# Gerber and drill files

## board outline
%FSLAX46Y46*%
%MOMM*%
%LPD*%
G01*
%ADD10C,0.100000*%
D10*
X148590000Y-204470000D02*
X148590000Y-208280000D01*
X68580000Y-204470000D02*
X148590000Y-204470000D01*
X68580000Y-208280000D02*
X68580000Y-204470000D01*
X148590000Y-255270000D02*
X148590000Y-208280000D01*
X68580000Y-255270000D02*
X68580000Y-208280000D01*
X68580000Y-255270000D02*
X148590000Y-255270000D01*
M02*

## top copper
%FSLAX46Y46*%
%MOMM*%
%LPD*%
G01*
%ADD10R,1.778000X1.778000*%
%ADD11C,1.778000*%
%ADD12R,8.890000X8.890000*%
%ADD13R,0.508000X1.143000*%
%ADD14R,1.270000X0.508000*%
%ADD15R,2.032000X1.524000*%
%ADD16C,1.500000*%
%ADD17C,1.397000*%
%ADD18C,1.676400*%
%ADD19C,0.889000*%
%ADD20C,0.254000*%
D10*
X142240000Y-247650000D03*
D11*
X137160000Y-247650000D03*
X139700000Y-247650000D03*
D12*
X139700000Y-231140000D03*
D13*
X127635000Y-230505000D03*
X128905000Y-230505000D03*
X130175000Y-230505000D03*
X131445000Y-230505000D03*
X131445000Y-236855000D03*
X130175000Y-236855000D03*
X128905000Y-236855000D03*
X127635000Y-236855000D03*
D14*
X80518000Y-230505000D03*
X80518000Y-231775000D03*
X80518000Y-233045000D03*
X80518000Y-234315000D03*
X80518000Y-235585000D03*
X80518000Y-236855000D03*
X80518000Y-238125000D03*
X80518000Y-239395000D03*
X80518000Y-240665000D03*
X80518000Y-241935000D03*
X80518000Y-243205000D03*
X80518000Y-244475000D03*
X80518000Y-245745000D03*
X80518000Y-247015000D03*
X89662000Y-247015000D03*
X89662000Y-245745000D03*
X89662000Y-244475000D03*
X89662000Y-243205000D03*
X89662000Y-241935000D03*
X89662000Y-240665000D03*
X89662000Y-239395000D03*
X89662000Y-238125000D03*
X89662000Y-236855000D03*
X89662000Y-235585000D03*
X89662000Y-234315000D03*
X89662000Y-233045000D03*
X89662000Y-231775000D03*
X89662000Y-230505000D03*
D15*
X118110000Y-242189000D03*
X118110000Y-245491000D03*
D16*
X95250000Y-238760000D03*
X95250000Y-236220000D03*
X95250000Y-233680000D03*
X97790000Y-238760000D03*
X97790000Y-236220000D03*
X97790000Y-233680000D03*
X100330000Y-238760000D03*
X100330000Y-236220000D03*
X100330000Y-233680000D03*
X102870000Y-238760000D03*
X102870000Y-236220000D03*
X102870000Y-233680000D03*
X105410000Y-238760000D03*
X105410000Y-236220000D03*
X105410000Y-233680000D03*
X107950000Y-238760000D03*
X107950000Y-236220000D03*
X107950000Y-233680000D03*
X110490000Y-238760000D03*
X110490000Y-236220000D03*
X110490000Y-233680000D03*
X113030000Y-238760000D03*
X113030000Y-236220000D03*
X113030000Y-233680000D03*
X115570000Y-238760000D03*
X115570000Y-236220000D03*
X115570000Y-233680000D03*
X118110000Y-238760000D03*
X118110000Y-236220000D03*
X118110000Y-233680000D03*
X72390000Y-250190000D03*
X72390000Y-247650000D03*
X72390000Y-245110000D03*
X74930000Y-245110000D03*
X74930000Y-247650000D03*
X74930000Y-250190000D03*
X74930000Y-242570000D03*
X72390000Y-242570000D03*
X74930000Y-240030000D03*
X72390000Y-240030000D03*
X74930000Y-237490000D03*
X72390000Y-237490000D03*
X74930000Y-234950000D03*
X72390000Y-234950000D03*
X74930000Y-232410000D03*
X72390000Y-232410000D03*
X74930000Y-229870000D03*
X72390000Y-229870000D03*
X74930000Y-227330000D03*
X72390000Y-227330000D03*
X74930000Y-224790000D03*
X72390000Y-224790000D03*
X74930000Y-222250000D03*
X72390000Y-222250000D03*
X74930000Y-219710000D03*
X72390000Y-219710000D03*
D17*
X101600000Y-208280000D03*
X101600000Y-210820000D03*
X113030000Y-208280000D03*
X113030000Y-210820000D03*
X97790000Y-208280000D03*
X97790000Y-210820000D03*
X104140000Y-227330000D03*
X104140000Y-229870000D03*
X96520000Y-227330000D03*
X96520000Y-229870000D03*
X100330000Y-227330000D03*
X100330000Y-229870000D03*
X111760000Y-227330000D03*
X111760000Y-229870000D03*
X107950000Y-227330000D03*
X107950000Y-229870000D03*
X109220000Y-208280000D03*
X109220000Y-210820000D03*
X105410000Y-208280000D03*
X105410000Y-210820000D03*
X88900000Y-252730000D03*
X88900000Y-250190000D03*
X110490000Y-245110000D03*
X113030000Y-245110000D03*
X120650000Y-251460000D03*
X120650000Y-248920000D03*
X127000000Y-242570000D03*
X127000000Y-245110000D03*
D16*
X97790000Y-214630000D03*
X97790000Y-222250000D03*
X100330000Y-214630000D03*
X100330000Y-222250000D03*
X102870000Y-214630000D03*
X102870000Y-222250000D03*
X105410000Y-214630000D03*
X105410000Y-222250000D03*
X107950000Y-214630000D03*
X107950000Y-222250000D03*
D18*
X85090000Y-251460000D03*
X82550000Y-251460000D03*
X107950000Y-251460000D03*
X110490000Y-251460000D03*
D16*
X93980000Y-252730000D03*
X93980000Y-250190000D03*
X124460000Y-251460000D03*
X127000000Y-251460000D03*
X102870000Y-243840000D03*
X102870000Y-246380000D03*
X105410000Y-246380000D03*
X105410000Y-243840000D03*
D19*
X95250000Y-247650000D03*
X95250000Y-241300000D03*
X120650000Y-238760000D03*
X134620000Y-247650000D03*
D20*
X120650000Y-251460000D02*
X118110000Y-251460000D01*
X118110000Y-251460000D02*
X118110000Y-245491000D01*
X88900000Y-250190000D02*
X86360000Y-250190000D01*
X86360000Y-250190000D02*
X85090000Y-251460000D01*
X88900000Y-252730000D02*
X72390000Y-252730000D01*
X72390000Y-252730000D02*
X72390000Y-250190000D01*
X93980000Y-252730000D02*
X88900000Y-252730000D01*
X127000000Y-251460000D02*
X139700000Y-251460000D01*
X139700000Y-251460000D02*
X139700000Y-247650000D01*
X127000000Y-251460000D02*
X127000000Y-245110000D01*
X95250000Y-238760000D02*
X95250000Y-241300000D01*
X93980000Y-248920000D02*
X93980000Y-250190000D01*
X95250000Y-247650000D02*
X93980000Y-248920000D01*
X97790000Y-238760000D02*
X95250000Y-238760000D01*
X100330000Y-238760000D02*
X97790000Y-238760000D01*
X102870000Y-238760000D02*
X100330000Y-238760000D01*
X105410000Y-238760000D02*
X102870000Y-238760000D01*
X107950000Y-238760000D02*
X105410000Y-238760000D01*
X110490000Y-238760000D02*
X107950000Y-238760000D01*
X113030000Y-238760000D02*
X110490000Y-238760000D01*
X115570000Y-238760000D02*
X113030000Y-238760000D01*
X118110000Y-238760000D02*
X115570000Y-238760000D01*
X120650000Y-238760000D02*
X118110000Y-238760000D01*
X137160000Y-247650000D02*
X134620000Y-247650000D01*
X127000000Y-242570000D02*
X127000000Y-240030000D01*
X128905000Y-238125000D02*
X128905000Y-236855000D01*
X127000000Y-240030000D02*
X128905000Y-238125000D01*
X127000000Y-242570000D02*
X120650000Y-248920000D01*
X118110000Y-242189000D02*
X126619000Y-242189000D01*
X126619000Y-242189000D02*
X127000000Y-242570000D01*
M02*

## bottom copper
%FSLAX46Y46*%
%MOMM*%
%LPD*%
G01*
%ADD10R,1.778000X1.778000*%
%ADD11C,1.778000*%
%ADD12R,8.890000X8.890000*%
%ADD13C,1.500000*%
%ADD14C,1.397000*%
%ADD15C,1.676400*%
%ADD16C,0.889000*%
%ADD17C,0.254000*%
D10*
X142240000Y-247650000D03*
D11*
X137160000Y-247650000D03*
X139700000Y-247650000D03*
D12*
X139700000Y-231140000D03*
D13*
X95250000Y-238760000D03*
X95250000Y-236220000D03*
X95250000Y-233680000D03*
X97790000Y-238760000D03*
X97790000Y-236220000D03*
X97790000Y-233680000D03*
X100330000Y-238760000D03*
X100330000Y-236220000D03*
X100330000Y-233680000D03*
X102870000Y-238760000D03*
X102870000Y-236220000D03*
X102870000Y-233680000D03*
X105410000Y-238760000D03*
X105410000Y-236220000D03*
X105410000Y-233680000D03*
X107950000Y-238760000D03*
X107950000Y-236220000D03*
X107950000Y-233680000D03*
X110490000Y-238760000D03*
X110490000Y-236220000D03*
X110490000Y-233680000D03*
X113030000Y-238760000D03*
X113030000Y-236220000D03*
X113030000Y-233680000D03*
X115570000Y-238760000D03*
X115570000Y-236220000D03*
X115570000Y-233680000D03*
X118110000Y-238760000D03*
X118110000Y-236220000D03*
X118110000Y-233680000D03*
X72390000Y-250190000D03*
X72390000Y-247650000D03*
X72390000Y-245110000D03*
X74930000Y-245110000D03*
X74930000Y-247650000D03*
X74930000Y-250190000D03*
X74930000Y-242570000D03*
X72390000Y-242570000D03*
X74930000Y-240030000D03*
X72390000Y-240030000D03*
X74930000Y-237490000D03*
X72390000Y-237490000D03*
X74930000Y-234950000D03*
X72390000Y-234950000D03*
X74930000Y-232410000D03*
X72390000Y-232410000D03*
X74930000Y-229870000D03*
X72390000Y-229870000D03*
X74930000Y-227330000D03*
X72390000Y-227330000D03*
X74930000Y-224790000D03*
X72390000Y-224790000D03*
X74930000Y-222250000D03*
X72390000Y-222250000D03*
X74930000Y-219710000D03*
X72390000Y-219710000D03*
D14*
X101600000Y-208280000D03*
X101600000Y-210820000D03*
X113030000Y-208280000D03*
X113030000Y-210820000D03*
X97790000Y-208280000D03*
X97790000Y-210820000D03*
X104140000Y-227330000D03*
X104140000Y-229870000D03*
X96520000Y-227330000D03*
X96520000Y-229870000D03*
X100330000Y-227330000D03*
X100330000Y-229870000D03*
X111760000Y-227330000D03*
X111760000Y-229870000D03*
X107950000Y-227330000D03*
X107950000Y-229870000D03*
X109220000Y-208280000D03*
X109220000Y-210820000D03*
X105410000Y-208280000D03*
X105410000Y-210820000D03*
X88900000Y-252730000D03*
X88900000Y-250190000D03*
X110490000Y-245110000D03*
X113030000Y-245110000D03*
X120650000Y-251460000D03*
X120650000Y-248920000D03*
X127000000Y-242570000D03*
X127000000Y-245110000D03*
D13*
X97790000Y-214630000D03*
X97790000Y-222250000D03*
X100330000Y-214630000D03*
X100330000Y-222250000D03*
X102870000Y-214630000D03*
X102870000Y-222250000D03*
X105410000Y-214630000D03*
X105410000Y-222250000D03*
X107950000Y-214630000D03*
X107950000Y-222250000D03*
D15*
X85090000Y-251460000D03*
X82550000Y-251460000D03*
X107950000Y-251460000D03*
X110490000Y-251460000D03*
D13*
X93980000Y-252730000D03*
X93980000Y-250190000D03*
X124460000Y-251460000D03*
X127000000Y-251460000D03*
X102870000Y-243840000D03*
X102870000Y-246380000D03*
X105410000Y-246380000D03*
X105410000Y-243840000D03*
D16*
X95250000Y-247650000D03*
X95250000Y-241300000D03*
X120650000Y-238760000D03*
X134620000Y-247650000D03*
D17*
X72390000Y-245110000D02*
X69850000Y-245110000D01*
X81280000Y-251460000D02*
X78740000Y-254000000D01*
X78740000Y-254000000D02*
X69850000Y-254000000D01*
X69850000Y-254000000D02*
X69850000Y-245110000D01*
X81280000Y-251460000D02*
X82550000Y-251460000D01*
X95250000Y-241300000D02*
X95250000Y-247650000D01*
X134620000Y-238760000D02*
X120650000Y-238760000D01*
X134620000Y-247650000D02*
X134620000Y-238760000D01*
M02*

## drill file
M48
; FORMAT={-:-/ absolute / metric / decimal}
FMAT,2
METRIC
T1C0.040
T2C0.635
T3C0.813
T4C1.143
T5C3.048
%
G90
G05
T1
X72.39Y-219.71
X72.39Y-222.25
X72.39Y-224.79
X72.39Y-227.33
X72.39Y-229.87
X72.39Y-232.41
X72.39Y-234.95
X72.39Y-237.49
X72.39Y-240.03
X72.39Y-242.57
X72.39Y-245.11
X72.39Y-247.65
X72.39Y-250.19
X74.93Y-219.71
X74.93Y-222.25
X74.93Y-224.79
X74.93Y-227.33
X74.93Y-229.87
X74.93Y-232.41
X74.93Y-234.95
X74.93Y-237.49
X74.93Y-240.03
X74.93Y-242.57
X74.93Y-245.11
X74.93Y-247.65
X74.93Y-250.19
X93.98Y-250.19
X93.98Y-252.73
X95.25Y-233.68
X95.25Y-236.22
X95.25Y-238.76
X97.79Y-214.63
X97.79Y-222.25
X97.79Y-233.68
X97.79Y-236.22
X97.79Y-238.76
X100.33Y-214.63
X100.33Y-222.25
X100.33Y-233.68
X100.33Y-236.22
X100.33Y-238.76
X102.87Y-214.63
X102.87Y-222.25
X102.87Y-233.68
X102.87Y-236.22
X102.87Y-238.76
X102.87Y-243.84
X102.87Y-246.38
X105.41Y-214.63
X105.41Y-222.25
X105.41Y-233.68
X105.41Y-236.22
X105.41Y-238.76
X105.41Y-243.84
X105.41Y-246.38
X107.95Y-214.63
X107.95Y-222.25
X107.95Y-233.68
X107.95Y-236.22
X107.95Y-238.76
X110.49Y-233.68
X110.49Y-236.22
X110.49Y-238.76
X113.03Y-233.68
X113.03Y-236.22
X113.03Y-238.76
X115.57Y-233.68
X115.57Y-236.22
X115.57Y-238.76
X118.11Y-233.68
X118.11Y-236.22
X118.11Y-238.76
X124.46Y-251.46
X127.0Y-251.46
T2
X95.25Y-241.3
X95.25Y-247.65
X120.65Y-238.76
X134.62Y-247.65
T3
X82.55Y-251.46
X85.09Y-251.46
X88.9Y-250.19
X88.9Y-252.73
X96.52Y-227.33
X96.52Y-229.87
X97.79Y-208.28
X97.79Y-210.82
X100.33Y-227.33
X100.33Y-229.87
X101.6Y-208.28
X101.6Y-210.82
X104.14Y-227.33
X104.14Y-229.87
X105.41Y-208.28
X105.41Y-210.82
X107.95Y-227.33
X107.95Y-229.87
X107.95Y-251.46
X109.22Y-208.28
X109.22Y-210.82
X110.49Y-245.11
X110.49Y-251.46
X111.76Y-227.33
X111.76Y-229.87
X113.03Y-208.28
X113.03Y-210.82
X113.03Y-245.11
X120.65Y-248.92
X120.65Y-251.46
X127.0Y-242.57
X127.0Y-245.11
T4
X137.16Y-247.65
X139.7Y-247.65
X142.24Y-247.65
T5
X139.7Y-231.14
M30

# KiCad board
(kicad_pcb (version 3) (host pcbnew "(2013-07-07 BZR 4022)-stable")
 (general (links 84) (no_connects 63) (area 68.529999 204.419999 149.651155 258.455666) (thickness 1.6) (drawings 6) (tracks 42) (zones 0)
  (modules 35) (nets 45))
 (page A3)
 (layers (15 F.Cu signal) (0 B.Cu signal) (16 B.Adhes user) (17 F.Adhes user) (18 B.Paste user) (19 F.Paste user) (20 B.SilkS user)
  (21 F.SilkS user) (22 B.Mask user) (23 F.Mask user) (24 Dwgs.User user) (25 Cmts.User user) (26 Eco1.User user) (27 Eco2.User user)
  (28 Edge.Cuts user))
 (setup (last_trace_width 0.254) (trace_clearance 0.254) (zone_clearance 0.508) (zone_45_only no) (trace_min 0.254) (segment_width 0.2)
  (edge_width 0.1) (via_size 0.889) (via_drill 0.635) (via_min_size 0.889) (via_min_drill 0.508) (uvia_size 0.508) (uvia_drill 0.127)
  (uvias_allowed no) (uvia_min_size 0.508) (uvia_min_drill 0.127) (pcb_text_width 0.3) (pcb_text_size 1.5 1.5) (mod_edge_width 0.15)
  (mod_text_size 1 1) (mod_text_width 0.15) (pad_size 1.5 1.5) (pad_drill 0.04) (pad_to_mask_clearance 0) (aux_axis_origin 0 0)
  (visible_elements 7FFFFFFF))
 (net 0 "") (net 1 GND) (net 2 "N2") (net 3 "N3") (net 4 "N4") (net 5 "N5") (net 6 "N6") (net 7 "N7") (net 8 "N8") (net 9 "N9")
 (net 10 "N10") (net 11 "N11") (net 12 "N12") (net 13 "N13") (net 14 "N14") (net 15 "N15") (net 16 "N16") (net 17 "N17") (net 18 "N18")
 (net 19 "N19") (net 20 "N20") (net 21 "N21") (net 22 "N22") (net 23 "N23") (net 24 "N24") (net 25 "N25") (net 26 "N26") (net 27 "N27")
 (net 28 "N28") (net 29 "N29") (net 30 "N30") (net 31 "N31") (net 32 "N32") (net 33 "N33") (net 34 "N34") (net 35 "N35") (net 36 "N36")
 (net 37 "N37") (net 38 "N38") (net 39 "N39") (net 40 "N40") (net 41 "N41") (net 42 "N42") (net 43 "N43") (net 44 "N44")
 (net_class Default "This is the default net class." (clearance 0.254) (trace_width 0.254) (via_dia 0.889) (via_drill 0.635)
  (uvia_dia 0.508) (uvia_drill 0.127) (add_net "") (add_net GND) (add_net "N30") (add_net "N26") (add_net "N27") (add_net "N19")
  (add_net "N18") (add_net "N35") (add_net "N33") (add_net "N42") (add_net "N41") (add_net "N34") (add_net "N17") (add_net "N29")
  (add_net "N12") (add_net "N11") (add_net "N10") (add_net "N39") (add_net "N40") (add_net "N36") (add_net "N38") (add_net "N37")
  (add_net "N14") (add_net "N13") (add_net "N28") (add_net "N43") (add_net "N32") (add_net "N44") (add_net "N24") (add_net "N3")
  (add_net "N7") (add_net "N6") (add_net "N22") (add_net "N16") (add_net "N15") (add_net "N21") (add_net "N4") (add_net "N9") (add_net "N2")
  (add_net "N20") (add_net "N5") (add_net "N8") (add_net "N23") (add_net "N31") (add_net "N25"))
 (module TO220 (layer F.Cu) (at 139.7 247.65 90)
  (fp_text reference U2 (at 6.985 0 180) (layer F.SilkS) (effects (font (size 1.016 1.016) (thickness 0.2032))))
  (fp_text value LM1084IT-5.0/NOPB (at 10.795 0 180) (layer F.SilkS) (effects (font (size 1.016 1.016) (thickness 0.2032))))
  (pad 1 thru_hole rect (at 0 2.54 90) (size 1.778 1.778) (drill 1.143) (layers *.Cu *.Mask F.SilkS) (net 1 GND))
  (pad 2 thru_hole circle (at 0 -2.54 90) (size 1.778 1.778) (drill 1.143) (layers *.Cu *.Mask F.SilkS) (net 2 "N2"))
  (pad 3 thru_hole circle (at 0 0 90) (size 1.778 1.778) (drill 1.143) (layers *.Cu *.Mask F.SilkS) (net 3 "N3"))
  (pad 4 thru_hole rect (at 16.51 0 90) (size 8.89 8.89) (drill 3.048) (layers *.Cu *.SilkS *.Mask)))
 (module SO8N (layer F.Cu) (at 129.54 233.68)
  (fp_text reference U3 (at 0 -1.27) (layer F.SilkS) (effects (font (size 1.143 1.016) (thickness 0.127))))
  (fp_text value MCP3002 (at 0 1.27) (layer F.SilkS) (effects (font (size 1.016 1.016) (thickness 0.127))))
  (pad 8 smd rect (at -1.905 -3.175) (size 0.508 1.143) (layers F.Cu F.Paste F.Mask) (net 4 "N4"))
  (pad 7 smd rect (at -0.635 -3.175) (size 0.508 1.143) (layers F.Cu F.Paste F.Mask) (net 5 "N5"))
  (pad 6 smd rect (at 0.635 -3.175) (size 0.508 1.143) (layers F.Cu F.Paste F.Mask) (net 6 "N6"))
  (pad 5 smd rect (at 1.905 -3.175) (size 0.508 1.143) (layers F.Cu F.Paste F.Mask) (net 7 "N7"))
  (pad 4 smd rect (at 1.905 3.175) (size 0.508 1.143) (layers F.Cu F.Paste F.Mask) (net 1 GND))
  (pad 3 smd rect (at 0.635 3.175) (size 0.508 1.143) (layers F.Cu F.Paste F.Mask))
  (pad 2 smd rect (at -0.635 3.175) (size 0.508 1.143) (layers F.Cu F.Paste F.Mask) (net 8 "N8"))
  (pad 1 smd rect (at -1.905 3.175) (size 0.508 1.143) (layers F.Cu F.Paste F.Mask) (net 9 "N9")))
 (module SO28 (layer F.Cu) (at 85.09 238.76 270)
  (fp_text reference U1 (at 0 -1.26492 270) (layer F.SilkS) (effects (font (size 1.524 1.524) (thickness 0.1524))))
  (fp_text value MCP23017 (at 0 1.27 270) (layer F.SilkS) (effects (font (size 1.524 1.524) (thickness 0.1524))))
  (pad 1 smd rect (at -8.255 4.572 270) (size 0.508 1.27) (layers F.Cu F.Paste F.Mask) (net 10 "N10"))
  (pad 2 smd rect (at -6.985 4.572 270) (size 0.508 1.27) (layers F.Cu F.Paste F.Mask) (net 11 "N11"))
  (pad 3 smd rect (at -5.715 4.572 270) (size 0.508 1.27) (layers F.Cu F.Paste F.Mask) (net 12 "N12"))
  (pad 4 smd rect (at -4.445 4.572 270) (size 0.508 1.27) (layers F.Cu F.Paste F.Mask) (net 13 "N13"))
  (pad 5 smd rect (at -3.175 4.572 270) (size 0.508 1.27) (layers F.Cu F.Paste F.Mask) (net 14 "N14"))
  (pad 6 smd rect (at -1.905 4.572 270) (size 0.508 1.27) (layers F.Cu F.Paste F.Mask))
  (pad 7 smd rect (at -0.635 4.572 270) (size 0.508 1.27) (layers F.Cu F.Paste F.Mask))
  (pad 8 smd rect (at 0.635 4.572 270) (size 0.508 1.27) (layers F.Cu F.Paste F.Mask))
  (pad 9 smd rect (at 1.905 4.572 270) (size 0.508 1.27) (layers F.Cu F.Paste F.Mask) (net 4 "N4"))
  (pad 10 smd rect (at 3.175 4.572 270) (size 0.508 1.27) (layers F.Cu F.Paste F.Mask) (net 1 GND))
  (pad 11 smd rect (at 4.445 4.572 270) (size 0.508 1.27) (layers F.Cu F.Paste F.Mask))
  (pad 12 smd rect (at 5.715 4.572 270) (size 0.508 1.27) (layers F.Cu F.Paste F.Mask) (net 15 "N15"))
  (pad 13 smd rect (at 6.985 4.572 270) (size 0.508 1.27) (layers F.Cu F.Paste F.Mask) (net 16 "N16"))
  (pad 14 smd rect (at 8.255 4.572 270) (size 0.508 1.27) (layers F.Cu F.Paste F.Mask))
  (pad 15 smd rect (at 8.255 -4.572 270) (size 0.508 1.27) (layers F.Cu F.Paste F.Mask) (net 1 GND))
  (pad 16 smd rect (at 6.985 -4.572 270) (size 0.508 1.27) (layers F.Cu F.Paste F.Mask) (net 1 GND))
  (pad 17 smd rect (at 5.715 -4.572 270) (size 0.508 1.27) (layers F.Cu F.Paste F.Mask) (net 1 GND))
  (pad 18 smd rect (at 4.445 -4.572 270) (size 0.508 1.27) (layers F.Cu F.Paste F.Mask) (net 4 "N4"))
  (pad 19 smd rect (at 3.175 -4.572 270) (size 0.508 1.27) (layers F.Cu F.Paste F.Mask))
  (pad 20 smd rect (at 1.905 -4.572 270) (size 0.508 1.27) (layers F.Cu F.Paste F.Mask))
  (pad 21 smd rect (at 0.635 -4.572 270) (size 0.508 1.27) (layers F.Cu F.Paste F.Mask) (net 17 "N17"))
  (pad 22 smd rect (at -0.635 -4.572 270) (size 0.508 1.27) (layers F.Cu F.Paste F.Mask) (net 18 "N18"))
  (pad 23 smd rect (at -1.905 -4.572 270) (size 0.508 1.27) (layers F.Cu F.Paste F.Mask) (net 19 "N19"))
  (pad 24 smd rect (at -3.175 -4.572 270) (size 0.508 1.27) (layers F.Cu F.Paste F.Mask) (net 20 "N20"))
  (pad 25 smd rect (at -4.445 -4.572 270) (size 0.508 1.27) (layers F.Cu F.Paste F.Mask) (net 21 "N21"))
  (pad 26 smd rect (at -5.715 -4.572 270) (size 0.508 1.27) (layers F.Cu F.Paste F.Mask))
  (pad 27 smd rect (at -6.985 -4.572 270) (size 0.508 1.27) (layers F.Cu F.Paste F.Mask))
  (pad 28 smd rect (at -8.255 -4.572 270) (size 0.508 1.27) (layers F.Cu F.Paste F.Mask)))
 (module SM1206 (layer F.Cu) (at 118.11 243.84 270)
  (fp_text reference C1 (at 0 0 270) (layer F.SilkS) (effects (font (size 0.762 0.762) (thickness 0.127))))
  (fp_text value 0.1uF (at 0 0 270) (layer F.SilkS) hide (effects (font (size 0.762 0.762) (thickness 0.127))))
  (pad 1 smd rect (at -1.651 0 270) (size 1.524 2.032) (layers F.Cu F.Paste F.Mask) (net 8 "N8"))
  (pad 2 smd rect (at 1.651 0 270) (size 1.524 2.032) (layers F.Cu F.Paste F.Mask) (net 1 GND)))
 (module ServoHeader (layer F.Cu) (at 95.25 234.95 90)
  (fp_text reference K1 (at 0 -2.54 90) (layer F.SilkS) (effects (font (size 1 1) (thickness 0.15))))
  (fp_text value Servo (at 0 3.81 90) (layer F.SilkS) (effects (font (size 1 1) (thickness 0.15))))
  (pad 1 thru_hole circle (at -3.81 0 90) (size 1.5 1.5) (drill 0.04) (layers *.Cu *.Mask F.SilkS) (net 2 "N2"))
  (pad 2 thru_hole circle (at -1.27 0 90) (size 1.5 1.5) (drill 0.04) (layers *.Cu *.Mask F.SilkS) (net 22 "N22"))
  (pad 3 thru_hole circle (at 1.27 0 90) (size 1.5 1.5) (drill 0.04) (layers *.Cu *.Mask F.SilkS) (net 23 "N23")))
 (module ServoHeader (layer F.Cu) (at 97.79 234.95 90)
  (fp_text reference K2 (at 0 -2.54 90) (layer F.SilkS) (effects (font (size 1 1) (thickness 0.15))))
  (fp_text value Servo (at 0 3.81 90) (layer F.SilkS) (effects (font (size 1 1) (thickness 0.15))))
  (pad 1 thru_hole circle (at -3.81 0 90) (size 1.5 1.5) (drill 0.04) (layers *.Cu *.Mask F.SilkS) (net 2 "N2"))
  (pad 2 thru_hole circle (at -1.27 0 90) (size 1.5 1.5) (drill 0.04) (layers *.Cu *.Mask F.SilkS) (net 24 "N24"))
  (pad 3 thru_hole circle (at 1.27 0 90) (size 1.5 1.5) (drill 0.04) (layers *.Cu *.Mask F.SilkS) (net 23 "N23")))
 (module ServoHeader (layer F.Cu) (at 100.33 234.95 90)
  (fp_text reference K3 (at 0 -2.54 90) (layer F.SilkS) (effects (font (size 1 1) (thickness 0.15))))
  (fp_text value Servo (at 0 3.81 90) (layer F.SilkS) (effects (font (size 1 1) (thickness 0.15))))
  (pad 1 thru_hole circle (at -3.81 0 90) (size 1.5 1.5) (drill 0.04) (layers *.Cu *.Mask F.SilkS) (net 2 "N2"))
  (pad 2 thru_hole circle (at -1.27 0 90) (size 1.5 1.5) (drill 0.04) (layers *.Cu *.Mask F.SilkS) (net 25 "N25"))
  (pad 3 thru_hole circle (at 1.27 0 90) (size 1.5 1.5) (drill 0.04) (layers *.Cu *.Mask F.SilkS) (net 23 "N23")))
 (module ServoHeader (layer F.Cu) (at 102.87 234.95 90)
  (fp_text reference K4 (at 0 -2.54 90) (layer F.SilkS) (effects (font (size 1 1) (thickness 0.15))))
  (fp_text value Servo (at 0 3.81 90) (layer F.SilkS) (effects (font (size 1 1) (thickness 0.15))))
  (pad 1 thru_hole circle (at -3.81 0 90) (size 1.5 1.5) (drill 0.04) (layers *.Cu *.Mask F.SilkS) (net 2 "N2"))
  (pad 2 thru_hole circle (at -1.27 0 90) (size 1.5 1.5) (drill 0.04) (layers *.Cu *.Mask F.SilkS) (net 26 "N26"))
  (pad 3 thru_hole circle (at 1.27 0 90) (size 1.5 1.5) (drill 0.04) (layers *.Cu *.Mask F.SilkS) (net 23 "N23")))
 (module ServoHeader (layer F.Cu) (at 105.41 234.95 90)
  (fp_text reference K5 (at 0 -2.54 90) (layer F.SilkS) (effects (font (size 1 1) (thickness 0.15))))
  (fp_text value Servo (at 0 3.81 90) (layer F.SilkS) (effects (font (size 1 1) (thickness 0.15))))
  (pad 1 thru_hole circle (at -3.81 0 90) (size 1.5 1.5) (drill 0.04) (layers *.Cu *.Mask F.SilkS) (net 2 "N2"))
  (pad 2 thru_hole circle (at -1.27 0 90) (size 1.5 1.5) (drill 0.04) (layers *.Cu *.Mask F.SilkS) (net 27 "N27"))
  (pad 3 thru_hole circle (at 1.27 0 90) (size 1.5 1.5) (drill 0.04) (layers *.Cu *.Mask F.SilkS) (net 23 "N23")))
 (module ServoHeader (layer F.Cu) (at 107.95 234.95 90)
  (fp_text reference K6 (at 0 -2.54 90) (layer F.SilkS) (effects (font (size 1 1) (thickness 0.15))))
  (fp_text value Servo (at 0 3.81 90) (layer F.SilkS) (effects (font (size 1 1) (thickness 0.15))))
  (pad 1 thru_hole circle (at -3.81 0 90) (size 1.5 1.5) (drill 0.04) (layers *.Cu *.Mask F.SilkS) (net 2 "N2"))
  (pad 2 thru_hole circle (at -1.27 0 90) (size 1.5 1.5) (drill 0.04) (layers *.Cu *.Mask F.SilkS) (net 23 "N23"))
  (pad 3 thru_hole circle (at 1.27 0 90) (size 1.5 1.5) (drill 0.04) (layers *.Cu *.Mask F.SilkS) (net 1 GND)))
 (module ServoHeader (layer F.Cu) (at 110.49 234.95 90)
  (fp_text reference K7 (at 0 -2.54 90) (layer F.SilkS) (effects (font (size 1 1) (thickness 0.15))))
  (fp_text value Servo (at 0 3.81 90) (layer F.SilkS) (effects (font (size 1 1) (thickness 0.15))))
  (pad 1 thru_hole circle (at -3.81 0 90) (size 1.5 1.5) (drill 0.04) (layers *.Cu *.Mask F.SilkS) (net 2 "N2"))
  (pad 2 thru_hole circle (at -1.27 0 90) (size 1.5 1.5) (drill 0.04) (layers *.Cu *.Mask F.SilkS) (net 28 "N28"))
  (pad 3 thru_hole circle (at 1.27 0 90) (size 1.5 1.5) (drill 0.04) (layers *.Cu *.Mask F.SilkS) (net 1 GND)))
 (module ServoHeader (layer F.Cu) (at 113.03 234.95 90)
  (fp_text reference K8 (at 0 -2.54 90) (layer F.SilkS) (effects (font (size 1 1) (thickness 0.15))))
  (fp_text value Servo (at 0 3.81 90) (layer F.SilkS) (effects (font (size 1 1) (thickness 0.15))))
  (pad 1 thru_hole circle (at -3.81 0 90) (size 1.5 1.5) (drill 0.04) (layers *.Cu *.Mask F.SilkS) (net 2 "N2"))
  (pad 2 thru_hole circle (at -1.27 0 90) (size 1.5 1.5) (drill 0.04) (layers *.Cu *.Mask F.SilkS) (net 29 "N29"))
  (pad 3 thru_hole circle (at 1.27 0 90) (size 1.5 1.5) (drill 0.04) (layers *.Cu *.Mask F.SilkS) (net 1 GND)))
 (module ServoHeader (layer F.Cu) (at 115.57 234.95 90)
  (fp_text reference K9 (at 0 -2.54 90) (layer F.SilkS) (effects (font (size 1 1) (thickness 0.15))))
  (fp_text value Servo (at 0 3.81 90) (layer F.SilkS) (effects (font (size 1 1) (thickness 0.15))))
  (pad 1 thru_hole circle (at -3.81 0 90) (size 1.5 1.5) (drill 0.04) (layers *.Cu *.Mask F.SilkS) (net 2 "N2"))
  (pad 2 thru_hole circle (at -1.27 0 90) (size 1.5 1.5) (drill 0.04) (layers *.Cu *.Mask F.SilkS) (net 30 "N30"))
  (pad 3 thru_hole circle (at 1.27 0 90) (size 1.5 1.5) (drill 0.04) (layers *.Cu *.Mask F.SilkS) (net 1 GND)))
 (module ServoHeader (layer F.Cu) (at 118.11 234.95 90)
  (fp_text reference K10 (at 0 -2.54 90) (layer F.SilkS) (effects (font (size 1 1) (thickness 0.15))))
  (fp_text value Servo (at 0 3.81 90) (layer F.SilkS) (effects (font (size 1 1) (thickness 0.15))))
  (pad 1 thru_hole circle (at -3.81 0 90) (size 1.5 1.5) (drill 0.04) (layers *.Cu *.Mask F.SilkS) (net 2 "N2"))
  (pad 2 thru_hole circle (at -1.27 0 90) (size 1.5 1.5) (drill 0.04) (layers *.Cu *.Mask F.SilkS) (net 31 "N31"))
  (pad 3 thru_hole circle (at 1.27 0 90) (size 1.5 1.5) (drill 0.04) (layers *.Cu *.Mask F.SilkS) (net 1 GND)))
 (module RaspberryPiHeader (layer F.Cu) (at 73.66 243.84 90)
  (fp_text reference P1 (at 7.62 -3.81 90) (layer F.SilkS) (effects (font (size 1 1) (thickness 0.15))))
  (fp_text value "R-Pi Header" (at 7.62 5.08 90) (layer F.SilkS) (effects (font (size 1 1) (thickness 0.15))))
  (pad 2 thru_hole circle (at -6.35 -1.27 90) (size 1.5 1.5) (drill 0.04) (layers *.Cu *.Mask F.SilkS) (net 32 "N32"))
  (pad 4 thru_hole circle (at -3.81 -1.27 90) (size 1.5 1.5) (drill 0.04) (layers *.Cu *.Mask F.SilkS))
  (pad 6 thru_hole circle (at -1.27 -1.27 90) (size 1.5 1.5) (drill 0.04) (layers *.Cu *.Mask F.SilkS) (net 1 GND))
  (pad 5 thru_hole circle (at -1.27 1.27 90) (size 1.5 1.5) (drill 0.04) (layers *.Cu *.Mask F.SilkS) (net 15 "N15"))
  (pad 3 thru_hole circle (at -3.81 1.27 90) (size 1.5 1.5) (drill 0.04) (layers *.Cu *.Mask F.SilkS) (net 16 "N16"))
  (pad 1 thru_hole circle (at -6.35 1.27 90) (size 1.5 1.5) (drill 0.04) (layers *.Cu *.Mask F.SilkS) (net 4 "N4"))
  (pad 7 thru_hole circle (at 1.27 1.27 90) (size 1.5 1.5) (drill 0.04) (layers *.Cu *.Mask F.SilkS) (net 31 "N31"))
  (pad 8 thru_hole circle (at 1.27 -1.27 90) (size 1.5 1.5) (drill 0.04) (layers *.Cu *.Mask F.SilkS) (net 23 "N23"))
  (pad 9 thru_hole circle (at 3.81 1.27 90) (size 1.5 1.5) (drill 0.04) (layers *.Cu *.Mask F.SilkS))
  (pad 10 thru_hole circle (at 3.81 -1.27 90) (size 1.5 1.5) (drill 0.04) (layers *.Cu *.Mask F.SilkS) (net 28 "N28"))
  (pad 11 thru_hole circle (at 6.35 1.27 90) (size 1.5 1.5) (drill 0.04) (layers *.Cu *.Mask F.SilkS) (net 27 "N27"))
  (pad 12 thru_hole circle (at 6.35 -1.27 90) (size 1.5 1.5) (drill 0.04) (layers *.Cu *.Mask F.SilkS) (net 29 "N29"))
  (pad 13 thru_hole circle (at 8.89 1.27 90) (size 1.5 1.5) (drill 0.04) (layers *.Cu *.Mask F.SilkS) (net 26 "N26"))
  (pad 14 thru_hole circle (at 8.89 -1.27 90) (size 1.5 1.5) (drill 0.04) (layers *.Cu *.Mask F.SilkS))
  (pad 15 thru_hole circle (at 11.43 1.27 90) (size 1.5 1.5) (drill 0.04) (layers *.Cu *.Mask F.SilkS) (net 25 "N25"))
  (pad 16 thru_hole circle (at 11.43 -1.27 90) (size 1.5 1.5) (drill 0.04) (layers *.Cu *.Mask F.SilkS) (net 6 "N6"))
  (pad 17 thru_hole circle (at 13.97 1.27 90) (size 1.5 1.5) (drill 0.04) (layers *.Cu *.Mask F.SilkS))
  (pad 18 thru_hole circle (at 13.97 -1.27 90) (size 1.5 1.5) (drill 0.04) (layers *.Cu *.Mask F.SilkS) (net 7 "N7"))
  (pad 19 thru_hole circle (at 16.51 1.27 90) (size 1.5 1.5) (drill 0.04) (layers *.Cu *.Mask F.SilkS) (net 24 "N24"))
  (pad 20 thru_hole circle (at 16.51 -1.27 90) (size 1.5 1.5) (drill 0.04) (layers *.Cu *.Mask F.SilkS))
  (pad 21 thru_hole circle (at 19.05 1.27 90) (size 1.5 1.5) (drill 0.04) (layers *.Cu *.Mask F.SilkS) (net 22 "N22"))
  (pad 22 thru_hole circle (at 19.05 -1.27 90) (size 1.5 1.5) (drill 0.04) (layers *.Cu *.Mask F.SilkS) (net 9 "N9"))
  (pad 23 thru_hole circle (at 21.59 1.27 90) (size 1.5 1.5) (drill 0.04) (layers *.Cu *.Mask F.SilkS))
  (pad 24 thru_hole circle (at 21.59 -1.27 90) (size 1.5 1.5) (drill 0.04) (layers *.Cu *.Mask F.SilkS) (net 5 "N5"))
  (pad 25 thru_hole circle (at 24.13 1.27 90) (size 1.5 1.5) (drill 0.04) (layers *.Cu *.Mask F.SilkS))
  (pad 26 thru_hole circle (at 24.13 -1.27 90) (size 1.5 1.5) (drill 0.04) (layers *.Cu *.Mask F.SilkS) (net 30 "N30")))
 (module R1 (layer F.Cu) (at 101.6 209.55 270) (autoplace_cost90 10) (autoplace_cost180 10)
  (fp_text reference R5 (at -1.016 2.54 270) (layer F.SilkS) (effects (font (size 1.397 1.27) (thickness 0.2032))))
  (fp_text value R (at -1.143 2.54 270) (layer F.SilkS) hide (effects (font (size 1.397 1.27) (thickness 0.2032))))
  (pad 1 thru_hole circle (at -1.27 0 270) (size 1.397 1.397) (drill 0.8128) (layers *.Cu *.Mask F.SilkS) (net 20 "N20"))
  (pad 2 thru_hole circle (at 1.27 0 270) (size 1.397 1.397) (drill 0.8128) (layers *.Cu *.Mask F.SilkS) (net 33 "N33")))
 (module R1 (layer F.Cu) (at 113.03 209.55 270) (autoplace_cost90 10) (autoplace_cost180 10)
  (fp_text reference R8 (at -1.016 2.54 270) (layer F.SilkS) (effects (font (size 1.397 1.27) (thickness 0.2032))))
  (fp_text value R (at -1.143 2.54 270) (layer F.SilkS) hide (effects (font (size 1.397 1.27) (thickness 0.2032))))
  (pad 1 thru_hole circle (at -1.27 0 270) (size 1.397 1.397) (drill 0.8128) (layers *.Cu *.Mask F.SilkS) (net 17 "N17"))
  (pad 2 thru_hole circle (at 1.27 0 270) (size 1.397 1.397) (drill 0.8128) (layers *.Cu *.Mask F.SilkS) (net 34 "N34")))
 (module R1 (layer F.Cu) (at 97.79 209.55 270) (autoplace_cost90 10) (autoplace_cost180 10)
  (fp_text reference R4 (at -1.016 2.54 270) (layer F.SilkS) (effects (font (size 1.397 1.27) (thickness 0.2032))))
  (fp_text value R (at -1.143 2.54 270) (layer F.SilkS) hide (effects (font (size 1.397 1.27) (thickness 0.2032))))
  (pad 1 thru_hole circle (at -1.27 0 270) (size 1.397 1.397) (drill 0.8128) (layers *.Cu *.Mask F.SilkS) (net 21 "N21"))
  (pad 2 thru_hole circle (at 1.27 0 270) (size 1.397 1.397) (drill 0.8128) (layers *.Cu *.Mask F.SilkS) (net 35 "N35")))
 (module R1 (layer F.Cu) (at 104.14 228.6 270) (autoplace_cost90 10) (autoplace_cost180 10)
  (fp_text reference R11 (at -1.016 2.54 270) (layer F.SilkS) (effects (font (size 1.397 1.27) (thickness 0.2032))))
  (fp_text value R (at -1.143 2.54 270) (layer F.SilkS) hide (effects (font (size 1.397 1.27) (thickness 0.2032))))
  (pad 1 thru_hole circle (at -1.27 0 270) (size 1.397 1.397) (drill 0.8128) (layers *.Cu *.Mask F.SilkS) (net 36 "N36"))
  (pad 2 thru_hole circle (at 1.27 0 270) (size 1.397 1.397) (drill 0.8128) (layers *.Cu *.Mask F.SilkS) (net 12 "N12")))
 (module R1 (layer F.Cu) (at 96.52 228.6 270) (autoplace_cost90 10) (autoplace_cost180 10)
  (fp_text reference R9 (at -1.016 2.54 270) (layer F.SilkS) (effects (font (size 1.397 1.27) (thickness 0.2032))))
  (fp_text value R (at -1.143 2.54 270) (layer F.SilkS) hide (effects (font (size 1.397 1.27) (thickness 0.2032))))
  (pad 1 thru_hole circle (at -1.27 0 270) (size 1.397 1.397) (drill 0.8128) (layers *.Cu *.Mask F.SilkS) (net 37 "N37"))
  (pad 2 thru_hole circle (at 1.27 0 270) (size 1.397 1.397) (drill 0.8128) (layers *.Cu *.Mask F.SilkS) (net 14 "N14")))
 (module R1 (layer F.Cu) (at 100.33 228.6 270) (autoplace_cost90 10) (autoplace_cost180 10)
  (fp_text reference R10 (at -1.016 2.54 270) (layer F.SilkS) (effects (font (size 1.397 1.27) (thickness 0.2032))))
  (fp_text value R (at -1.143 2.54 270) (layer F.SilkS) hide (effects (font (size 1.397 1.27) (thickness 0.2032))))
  (pad 1 thru_hole circle (at -1.27 0 270) (size 1.397 1.397) (drill 0.8128) (layers *.Cu *.Mask F.SilkS) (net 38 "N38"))
  (pad 2 thru_hole circle (at 1.27 0 270) (size 1.397 1.397) (drill 0.8128) (layers *.Cu *.Mask F.SilkS) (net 13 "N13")))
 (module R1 (layer F.Cu) (at 111.76 228.6 270) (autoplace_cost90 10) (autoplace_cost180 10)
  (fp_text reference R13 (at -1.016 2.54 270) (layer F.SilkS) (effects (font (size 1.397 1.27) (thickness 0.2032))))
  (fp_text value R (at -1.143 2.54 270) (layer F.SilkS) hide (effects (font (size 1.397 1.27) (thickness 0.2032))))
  (pad 1 thru_hole circle (at -1.27 0 270) (size 1.397 1.397) (drill 0.8128) (layers *.Cu *.Mask F.SilkS) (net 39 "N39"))
  (pad 2 thru_hole circle (at 1.27 0 270) (size 1.397 1.397) (drill 0.8128) (layers *.Cu *.Mask F.SilkS) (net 10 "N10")))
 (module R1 (layer F.Cu) (at 107.95 228.6 270) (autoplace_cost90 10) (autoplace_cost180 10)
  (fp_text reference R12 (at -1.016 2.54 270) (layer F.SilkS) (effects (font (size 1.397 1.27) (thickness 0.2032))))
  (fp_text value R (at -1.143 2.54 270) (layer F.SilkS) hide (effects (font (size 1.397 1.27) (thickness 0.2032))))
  (pad 1 thru_hole circle (at -1.27 0 270) (size 1.397 1.397) (drill 0.8128) (layers *.Cu *.Mask F.SilkS) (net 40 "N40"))
  (pad 2 thru_hole circle (at 1.27 0 270) (size 1.397 1.397) (drill 0.8128) (layers *.Cu *.Mask F.SilkS) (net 11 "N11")))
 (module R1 (layer F.Cu) (at 109.22 209.55 270) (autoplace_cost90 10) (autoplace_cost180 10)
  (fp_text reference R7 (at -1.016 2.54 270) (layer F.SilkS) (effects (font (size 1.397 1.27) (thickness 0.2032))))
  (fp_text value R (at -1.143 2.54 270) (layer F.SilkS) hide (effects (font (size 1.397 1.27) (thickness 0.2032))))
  (pad 1 thru_hole circle (at -1.27 0 270) (size 1.397 1.397) (drill 0.8128) (layers *.Cu *.Mask F.SilkS) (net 18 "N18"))
  (pad 2 thru_hole circle (at 1.27 0 270) (size 1.397 1.397) (drill 0.8128) (layers *.Cu *.Mask F.SilkS) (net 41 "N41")))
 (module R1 (layer F.Cu) (at 105.41 209.55 270) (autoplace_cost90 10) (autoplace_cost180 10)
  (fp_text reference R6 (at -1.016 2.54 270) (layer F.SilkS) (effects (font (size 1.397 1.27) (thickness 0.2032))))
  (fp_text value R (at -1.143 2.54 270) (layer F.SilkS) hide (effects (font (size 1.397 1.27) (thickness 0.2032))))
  (pad 1 thru_hole circle (at -1.27 0 270) (size 1.397 1.397) (drill 0.8128) (layers *.Cu *.Mask F.SilkS) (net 19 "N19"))
  (pad 2 thru_hole circle (at 1.27 0 270) (size 1.397 1.397) (drill 0.8128) (layers *.Cu *.Mask F.SilkS) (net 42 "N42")))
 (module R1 (layer F.Cu) (at 88.9 251.46 90) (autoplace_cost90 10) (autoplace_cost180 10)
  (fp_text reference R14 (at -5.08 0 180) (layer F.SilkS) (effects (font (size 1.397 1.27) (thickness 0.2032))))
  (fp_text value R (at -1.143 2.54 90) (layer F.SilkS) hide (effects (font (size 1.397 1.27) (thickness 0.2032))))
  (pad 1 thru_hole circle (at -1.27 0 90) (size 1.397 1.397) (drill 0.8128) (layers *.Cu *.Mask F.SilkS) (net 32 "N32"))
  (pad 2 thru_hole circle (at 1.27 0 90) (size 1.397 1.397) (drill 0.8128) (layers *.Cu *.Mask F.SilkS) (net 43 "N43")))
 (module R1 (layer F.Cu) (at 111.76 245.11) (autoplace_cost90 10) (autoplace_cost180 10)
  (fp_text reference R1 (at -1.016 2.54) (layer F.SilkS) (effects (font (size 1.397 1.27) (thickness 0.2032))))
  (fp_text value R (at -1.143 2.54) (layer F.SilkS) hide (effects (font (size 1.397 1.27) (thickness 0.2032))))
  (pad 1 thru_hole circle (at -1.27 0) (size 1.397 1.397) (drill 0.8128) (layers *.Cu *.Mask F.SilkS) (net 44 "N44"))
  (pad 2 thru_hole circle (at 1.27 0) (size 1.397 1.397) (drill 0.8128) (layers *.Cu *.Mask F.SilkS) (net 2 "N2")))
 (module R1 (layer F.Cu) (at 120.65 250.19 90) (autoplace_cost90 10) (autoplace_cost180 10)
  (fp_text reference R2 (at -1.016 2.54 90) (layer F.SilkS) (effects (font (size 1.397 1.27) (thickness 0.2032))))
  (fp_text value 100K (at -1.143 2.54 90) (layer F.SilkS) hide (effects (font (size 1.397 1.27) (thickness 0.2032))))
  (pad 1 thru_hole circle (at -1.27 0 90) (size 1.397 1.397) (drill 0.8128) (layers *.Cu *.Mask F.SilkS) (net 1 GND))
  (pad 2 thru_hole circle (at 1.27 0 90) (size 1.397 1.397) (drill 0.8128) (layers *.Cu *.Mask F.SilkS) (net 8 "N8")))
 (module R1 (layer F.Cu) (at 127 243.84 270) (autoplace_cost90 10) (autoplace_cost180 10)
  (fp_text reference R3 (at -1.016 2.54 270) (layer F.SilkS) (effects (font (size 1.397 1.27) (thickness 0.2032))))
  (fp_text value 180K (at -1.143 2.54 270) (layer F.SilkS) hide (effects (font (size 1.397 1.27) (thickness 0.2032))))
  (pad 1 thru_hole circle (at -1.27 0 270) (size 1.397 1.397) (drill 0.8128) (layers *.Cu *.Mask F.SilkS) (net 8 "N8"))
  (pad 2 thru_hole circle (at 1.27 0 270) (size 1.397 1.397) (drill 0.8128) (layers *.Cu *.Mask F.SilkS) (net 3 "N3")))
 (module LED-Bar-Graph (layer F.Cu) (at 102.87 213.36)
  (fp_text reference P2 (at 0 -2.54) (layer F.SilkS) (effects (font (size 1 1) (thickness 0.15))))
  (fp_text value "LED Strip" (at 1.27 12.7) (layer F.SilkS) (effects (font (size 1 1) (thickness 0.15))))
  (pad 1 thru_hole circle (at -5.08 1.27) (size 1.5 1.5) (drill 0.04) (layers *.Cu *.Mask F.SilkS) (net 35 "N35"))
  (pad 2 thru_hole circle (at -5.08 8.89) (size 1.5 1.5) (drill 0.04) (layers *.Cu *.Mask F.SilkS) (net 37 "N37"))
  (pad 3 thru_hole circle (at -2.54 1.27) (size 1.5 1.5) (drill 0.04) (layers *.Cu *.Mask F.SilkS) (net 33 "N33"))
  (pad 4 thru_hole circle (at -2.54 8.89) (size 1.5 1.5) (drill 0.04) (layers *.Cu *.Mask F.SilkS) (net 38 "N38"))
  (pad 5 thru_hole circle (at 0 1.27) (size 1.5 1.5) (drill 0.04) (layers *.Cu *.Mask F.SilkS) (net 42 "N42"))
  (pad 6 thru_hole circle (at 0 8.89) (size 1.5 1.5) (drill 0.04) (layers *.Cu *.Mask F.SilkS) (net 36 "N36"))
  (pad 7 thru_hole circle (at 2.54 1.27) (size 1.5 1.5) (drill 0.04) (layers *.Cu *.Mask F.SilkS) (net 41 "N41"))
  (pad 8 thru_hole circle (at 2.54 8.89) (size 1.5 1.5) (drill 0.04) (layers *.Cu *.Mask F.SilkS) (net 40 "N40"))
  (pad 9 thru_hole circle (at 5.08 1.27) (size 1.5 1.5) (drill 0.04) (layers *.Cu *.Mask F.SilkS) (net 34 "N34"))
  (pad 10 thru_hole circle (at 5.08 8.89) (size 1.5 1.5) (drill 0.04) (layers *.Cu *.Mask F.SilkS) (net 39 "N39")))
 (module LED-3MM (layer F.Cu) (at 83.82 251.46 180)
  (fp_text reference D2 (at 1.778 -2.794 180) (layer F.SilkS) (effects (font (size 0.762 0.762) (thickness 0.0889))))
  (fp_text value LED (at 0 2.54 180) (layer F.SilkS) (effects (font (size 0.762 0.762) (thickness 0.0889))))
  (pad 1 thru_hole circle (at -1.27 0 180) (size 1.6764 1.6764) (drill 0.8128) (layers *.Cu *.Mask F.SilkS) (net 43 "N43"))
  (pad 2 thru_hole circle (at 1.27 0 180) (size 1.6764 1.6764) (drill 0.8128) (layers *.Cu *.Mask F.SilkS) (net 1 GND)))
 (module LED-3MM (layer F.Cu) (at 109.22 251.46)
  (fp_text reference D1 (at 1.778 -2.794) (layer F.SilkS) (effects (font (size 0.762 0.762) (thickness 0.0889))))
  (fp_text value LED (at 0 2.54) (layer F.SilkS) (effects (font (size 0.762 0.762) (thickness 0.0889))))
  (pad 1 thru_hole circle (at -1.27 0) (size 1.6764 1.6764) (drill 0.8128) (layers *.Cu *.Mask F.SilkS) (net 44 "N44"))
  (pad 2 thru_hole circle (at 1.27 0) (size 1.6764 1.6764) (drill 0.8128) (layers *.Cu *.Mask F.SilkS) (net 1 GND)))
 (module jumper (layer F.Cu) (at 93.98 251.46 90)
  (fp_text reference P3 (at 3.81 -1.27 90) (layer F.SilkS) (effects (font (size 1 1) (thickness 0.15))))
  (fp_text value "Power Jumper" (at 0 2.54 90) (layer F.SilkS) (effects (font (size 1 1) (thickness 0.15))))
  (pad 1 thru_hole circle (at -1.27 0 90) (size 1.5 1.5) (drill 0.04) (layers *.Cu *.Mask F.SilkS) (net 32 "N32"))
  (pad 2 thru_hole circle (at 1.27 0 90) (size 1.5 1.5) (drill 0.04) (layers *.Cu *.Mask F.SilkS) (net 2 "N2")))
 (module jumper (layer F.Cu) (at 125.73 251.46)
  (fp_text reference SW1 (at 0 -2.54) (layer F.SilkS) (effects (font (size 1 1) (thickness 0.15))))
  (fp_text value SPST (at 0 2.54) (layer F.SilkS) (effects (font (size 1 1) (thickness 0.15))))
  (pad 1 thru_hole circle (at -1.27 0) (size 1.5 1.5) (drill 0.04) (layers *.Cu *.Mask F.SilkS))
  (pad 2 thru_hole circle (at 1.27 0) (size 1.5 1.5) (drill 0.04) (layers *.Cu *.Mask F.SilkS) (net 3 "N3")))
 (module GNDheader (layer F.Cu) (at 105.41 242.57)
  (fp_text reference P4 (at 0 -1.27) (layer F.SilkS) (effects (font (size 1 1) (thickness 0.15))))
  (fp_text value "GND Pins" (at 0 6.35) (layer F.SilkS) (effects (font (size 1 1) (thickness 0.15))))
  (pad 1 thru_hole circle (at -2.54 1.27) (size 1.5 1.5) (drill 0.04) (layers *.Cu *.Mask F.SilkS) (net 1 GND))
  (pad 2 thru_hole circle (at -2.54 3.81) (size 1.5 1.5) (drill 0.04) (layers *.Cu *.Mask F.SilkS) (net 1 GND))
  (pad 4 thru_hole circle (at 0 3.81) (size 1.5 1.5) (drill 0.04) (layers *.Cu *.Mask F.SilkS) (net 1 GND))
  (pad 3 thru_hole circle (at 0 1.27) (size 1.5 1.5) (drill 0.04) (layers *.Cu *.Mask F.SilkS) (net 1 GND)))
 (gr_line (start 148.59 204.47) (end 148.59 208.28) (angle 90) (layer Edge.Cuts) (width 0.1))
 (gr_line (start 68.58 204.47) (end 148.59 204.47) (angle 90) (layer Edge.Cuts) (width 0.1))
 (gr_line (start 68.58 208.28) (end 68.58 204.47) (angle 90) (layer Edge.Cuts) (width 0.1))
 (gr_line (start 148.59 255.27) (end 148.59 208.28) (angle 90) (layer Edge.Cuts) (width 0.1))
 (gr_line (start 68.58 255.27) (end 68.58 208.28) (angle 90) (layer Edge.Cuts) (width 0.1))
 (gr_line (start 68.58 255.27) (end 148.59 255.27) (angle 90) (layer Edge.Cuts) (width 0.1))
 (segment (start 120.65 251.46) (end 118.11 251.46) (width 0.254) (layer F.Cu) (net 1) (status 400000))
 (segment (start 118.11 251.46) (end 118.11 245.491) (width 0.254) (layer F.Cu) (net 1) (status 800000))
 (segment (start 72.39 245.11) (end 69.85 245.11) (width 0.254) (layer B.Cu) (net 1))
 (segment (start 81.28 251.46) (end 78.74 254) (width 0.254) (layer B.Cu) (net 1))
 (segment (start 78.74 254) (end 69.85 254) (width 0.254) (layer B.Cu) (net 1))
 (segment (start 69.85 254) (end 69.85 245.11) (width 0.254) (layer B.Cu) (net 1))
 (segment (start 81.28 251.46) (end 82.55 251.46) (width 0.254) (layer B.Cu) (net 1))
 (segment (start 88.9 250.19) (end 86.36 250.19) (width 0.254) (layer F.Cu) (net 43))
 (segment (start 86.36 250.19) (end 85.09 251.46) (width 0.254) (layer F.Cu) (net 43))
 (segment (start 88.9 252.73) (end 72.39 252.73) (width 0.254) (layer F.Cu) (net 32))
 (segment (start 72.39 252.73) (end 72.39 250.19) (width 0.254) (layer F.Cu) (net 32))
 (segment (start 93.98 252.73) (end 88.9 252.73) (width 0.254) (layer F.Cu) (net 32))
 (segment (start 127 251.46) (end 139.7 251.46) (width 0.254) (layer F.Cu) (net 3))
 (segment (start 139.7 251.46) (end 139.7 247.65) (width 0.254) (layer F.Cu) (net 3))
 (segment (start 127 251.46) (end 127 245.11) (width 0.254) (layer F.Cu) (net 3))
 (segment (start 95.25 238.76) (end 95.25 241.3) (width 0.254) (layer F.Cu) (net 2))
 (segment (start 93.98 248.92) (end 93.98 250.19) (width 0.254) (layer F.Cu) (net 2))
 (segment (start 95.25 247.65) (end 93.98 248.92) (width 0.254) (layer F.Cu) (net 2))
 (via (at 95.25 247.65) (size 0.889) (layers F.Cu B.Cu) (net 2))
 (segment (start 95.25 241.3) (end 95.25 247.65) (width 0.254) (layer B.Cu) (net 2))
 (via (at 95.25 241.3) (size 0.889) (layers F.Cu B.Cu) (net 2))
 (segment (start 97.79 238.76) (end 95.25 238.76) (width 0.254) (layer F.Cu) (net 2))
 (segment (start 100.33 238.76) (end 97.79 238.76) (width 0.254) (layer F.Cu) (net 2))
 (segment (start 102.87 238.76) (end 100.33 238.76) (width 0.254) (layer F.Cu) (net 2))
 (segment (start 105.41 238.76) (end 102.87 238.76) (width 0.254) (layer F.Cu) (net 2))
 (segment (start 107.95 238.76) (end 105.41 238.76) (width 0.254) (layer F.Cu) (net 2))
 (segment (start 110.49 238.76) (end 107.95 238.76) (width 0.254) (layer F.Cu) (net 2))
 (segment (start 113.03 238.76) (end 110.49 238.76) (width 0.254) (layer F.Cu) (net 2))
 (segment (start 115.57 238.76) (end 113.03 238.76) (width 0.254) (layer F.Cu) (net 2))
 (segment (start 118.11 238.76) (end 115.57 238.76) (width 0.254) (layer F.Cu) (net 2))
 (segment (start 120.65 238.76) (end 118.11 238.76) (width 0.254) (layer F.Cu) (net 2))
 (segment (start 137.16 247.65) (end 134.62 247.65) (width 0.254) (layer F.Cu) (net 2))
 (via (at 120.65 238.76) (size 0.889) (layers F.Cu B.Cu) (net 2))
 (segment (start 134.62 238.76) (end 120.65 238.76) (width 0.254) (layer B.Cu) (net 2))
 (segment (start 134.62 247.65) (end 134.62 238.76) (width 0.254) (layer B.Cu) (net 2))
 (via (at 134.62 247.65) (size 0.889) (layers F.Cu B.Cu) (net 2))
 (segment (start 127 242.57) (end 127 240.03) (width 0.254) (layer F.Cu) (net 8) (status 400000))
 (segment (start 128.905 238.125) (end 128.905 236.855) (width 0.254) (layer F.Cu) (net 8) (status 800000))
 (segment (start 127 240.03) (end 128.905 238.125) (width 0.254) (layer F.Cu) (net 8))
 (segment (start 127 242.57) (end 120.65 248.92) (width 0.254) (layer F.Cu) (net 8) (status C00000))
 (segment (start 118.11 242.189) (end 126.619 242.189) (width 0.254) (layer F.Cu) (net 8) (status C00000))
 (segment (start 126.619 242.189) (end 127 242.57) (width 0.254) (layer F.Cu) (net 8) (status C00000)))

